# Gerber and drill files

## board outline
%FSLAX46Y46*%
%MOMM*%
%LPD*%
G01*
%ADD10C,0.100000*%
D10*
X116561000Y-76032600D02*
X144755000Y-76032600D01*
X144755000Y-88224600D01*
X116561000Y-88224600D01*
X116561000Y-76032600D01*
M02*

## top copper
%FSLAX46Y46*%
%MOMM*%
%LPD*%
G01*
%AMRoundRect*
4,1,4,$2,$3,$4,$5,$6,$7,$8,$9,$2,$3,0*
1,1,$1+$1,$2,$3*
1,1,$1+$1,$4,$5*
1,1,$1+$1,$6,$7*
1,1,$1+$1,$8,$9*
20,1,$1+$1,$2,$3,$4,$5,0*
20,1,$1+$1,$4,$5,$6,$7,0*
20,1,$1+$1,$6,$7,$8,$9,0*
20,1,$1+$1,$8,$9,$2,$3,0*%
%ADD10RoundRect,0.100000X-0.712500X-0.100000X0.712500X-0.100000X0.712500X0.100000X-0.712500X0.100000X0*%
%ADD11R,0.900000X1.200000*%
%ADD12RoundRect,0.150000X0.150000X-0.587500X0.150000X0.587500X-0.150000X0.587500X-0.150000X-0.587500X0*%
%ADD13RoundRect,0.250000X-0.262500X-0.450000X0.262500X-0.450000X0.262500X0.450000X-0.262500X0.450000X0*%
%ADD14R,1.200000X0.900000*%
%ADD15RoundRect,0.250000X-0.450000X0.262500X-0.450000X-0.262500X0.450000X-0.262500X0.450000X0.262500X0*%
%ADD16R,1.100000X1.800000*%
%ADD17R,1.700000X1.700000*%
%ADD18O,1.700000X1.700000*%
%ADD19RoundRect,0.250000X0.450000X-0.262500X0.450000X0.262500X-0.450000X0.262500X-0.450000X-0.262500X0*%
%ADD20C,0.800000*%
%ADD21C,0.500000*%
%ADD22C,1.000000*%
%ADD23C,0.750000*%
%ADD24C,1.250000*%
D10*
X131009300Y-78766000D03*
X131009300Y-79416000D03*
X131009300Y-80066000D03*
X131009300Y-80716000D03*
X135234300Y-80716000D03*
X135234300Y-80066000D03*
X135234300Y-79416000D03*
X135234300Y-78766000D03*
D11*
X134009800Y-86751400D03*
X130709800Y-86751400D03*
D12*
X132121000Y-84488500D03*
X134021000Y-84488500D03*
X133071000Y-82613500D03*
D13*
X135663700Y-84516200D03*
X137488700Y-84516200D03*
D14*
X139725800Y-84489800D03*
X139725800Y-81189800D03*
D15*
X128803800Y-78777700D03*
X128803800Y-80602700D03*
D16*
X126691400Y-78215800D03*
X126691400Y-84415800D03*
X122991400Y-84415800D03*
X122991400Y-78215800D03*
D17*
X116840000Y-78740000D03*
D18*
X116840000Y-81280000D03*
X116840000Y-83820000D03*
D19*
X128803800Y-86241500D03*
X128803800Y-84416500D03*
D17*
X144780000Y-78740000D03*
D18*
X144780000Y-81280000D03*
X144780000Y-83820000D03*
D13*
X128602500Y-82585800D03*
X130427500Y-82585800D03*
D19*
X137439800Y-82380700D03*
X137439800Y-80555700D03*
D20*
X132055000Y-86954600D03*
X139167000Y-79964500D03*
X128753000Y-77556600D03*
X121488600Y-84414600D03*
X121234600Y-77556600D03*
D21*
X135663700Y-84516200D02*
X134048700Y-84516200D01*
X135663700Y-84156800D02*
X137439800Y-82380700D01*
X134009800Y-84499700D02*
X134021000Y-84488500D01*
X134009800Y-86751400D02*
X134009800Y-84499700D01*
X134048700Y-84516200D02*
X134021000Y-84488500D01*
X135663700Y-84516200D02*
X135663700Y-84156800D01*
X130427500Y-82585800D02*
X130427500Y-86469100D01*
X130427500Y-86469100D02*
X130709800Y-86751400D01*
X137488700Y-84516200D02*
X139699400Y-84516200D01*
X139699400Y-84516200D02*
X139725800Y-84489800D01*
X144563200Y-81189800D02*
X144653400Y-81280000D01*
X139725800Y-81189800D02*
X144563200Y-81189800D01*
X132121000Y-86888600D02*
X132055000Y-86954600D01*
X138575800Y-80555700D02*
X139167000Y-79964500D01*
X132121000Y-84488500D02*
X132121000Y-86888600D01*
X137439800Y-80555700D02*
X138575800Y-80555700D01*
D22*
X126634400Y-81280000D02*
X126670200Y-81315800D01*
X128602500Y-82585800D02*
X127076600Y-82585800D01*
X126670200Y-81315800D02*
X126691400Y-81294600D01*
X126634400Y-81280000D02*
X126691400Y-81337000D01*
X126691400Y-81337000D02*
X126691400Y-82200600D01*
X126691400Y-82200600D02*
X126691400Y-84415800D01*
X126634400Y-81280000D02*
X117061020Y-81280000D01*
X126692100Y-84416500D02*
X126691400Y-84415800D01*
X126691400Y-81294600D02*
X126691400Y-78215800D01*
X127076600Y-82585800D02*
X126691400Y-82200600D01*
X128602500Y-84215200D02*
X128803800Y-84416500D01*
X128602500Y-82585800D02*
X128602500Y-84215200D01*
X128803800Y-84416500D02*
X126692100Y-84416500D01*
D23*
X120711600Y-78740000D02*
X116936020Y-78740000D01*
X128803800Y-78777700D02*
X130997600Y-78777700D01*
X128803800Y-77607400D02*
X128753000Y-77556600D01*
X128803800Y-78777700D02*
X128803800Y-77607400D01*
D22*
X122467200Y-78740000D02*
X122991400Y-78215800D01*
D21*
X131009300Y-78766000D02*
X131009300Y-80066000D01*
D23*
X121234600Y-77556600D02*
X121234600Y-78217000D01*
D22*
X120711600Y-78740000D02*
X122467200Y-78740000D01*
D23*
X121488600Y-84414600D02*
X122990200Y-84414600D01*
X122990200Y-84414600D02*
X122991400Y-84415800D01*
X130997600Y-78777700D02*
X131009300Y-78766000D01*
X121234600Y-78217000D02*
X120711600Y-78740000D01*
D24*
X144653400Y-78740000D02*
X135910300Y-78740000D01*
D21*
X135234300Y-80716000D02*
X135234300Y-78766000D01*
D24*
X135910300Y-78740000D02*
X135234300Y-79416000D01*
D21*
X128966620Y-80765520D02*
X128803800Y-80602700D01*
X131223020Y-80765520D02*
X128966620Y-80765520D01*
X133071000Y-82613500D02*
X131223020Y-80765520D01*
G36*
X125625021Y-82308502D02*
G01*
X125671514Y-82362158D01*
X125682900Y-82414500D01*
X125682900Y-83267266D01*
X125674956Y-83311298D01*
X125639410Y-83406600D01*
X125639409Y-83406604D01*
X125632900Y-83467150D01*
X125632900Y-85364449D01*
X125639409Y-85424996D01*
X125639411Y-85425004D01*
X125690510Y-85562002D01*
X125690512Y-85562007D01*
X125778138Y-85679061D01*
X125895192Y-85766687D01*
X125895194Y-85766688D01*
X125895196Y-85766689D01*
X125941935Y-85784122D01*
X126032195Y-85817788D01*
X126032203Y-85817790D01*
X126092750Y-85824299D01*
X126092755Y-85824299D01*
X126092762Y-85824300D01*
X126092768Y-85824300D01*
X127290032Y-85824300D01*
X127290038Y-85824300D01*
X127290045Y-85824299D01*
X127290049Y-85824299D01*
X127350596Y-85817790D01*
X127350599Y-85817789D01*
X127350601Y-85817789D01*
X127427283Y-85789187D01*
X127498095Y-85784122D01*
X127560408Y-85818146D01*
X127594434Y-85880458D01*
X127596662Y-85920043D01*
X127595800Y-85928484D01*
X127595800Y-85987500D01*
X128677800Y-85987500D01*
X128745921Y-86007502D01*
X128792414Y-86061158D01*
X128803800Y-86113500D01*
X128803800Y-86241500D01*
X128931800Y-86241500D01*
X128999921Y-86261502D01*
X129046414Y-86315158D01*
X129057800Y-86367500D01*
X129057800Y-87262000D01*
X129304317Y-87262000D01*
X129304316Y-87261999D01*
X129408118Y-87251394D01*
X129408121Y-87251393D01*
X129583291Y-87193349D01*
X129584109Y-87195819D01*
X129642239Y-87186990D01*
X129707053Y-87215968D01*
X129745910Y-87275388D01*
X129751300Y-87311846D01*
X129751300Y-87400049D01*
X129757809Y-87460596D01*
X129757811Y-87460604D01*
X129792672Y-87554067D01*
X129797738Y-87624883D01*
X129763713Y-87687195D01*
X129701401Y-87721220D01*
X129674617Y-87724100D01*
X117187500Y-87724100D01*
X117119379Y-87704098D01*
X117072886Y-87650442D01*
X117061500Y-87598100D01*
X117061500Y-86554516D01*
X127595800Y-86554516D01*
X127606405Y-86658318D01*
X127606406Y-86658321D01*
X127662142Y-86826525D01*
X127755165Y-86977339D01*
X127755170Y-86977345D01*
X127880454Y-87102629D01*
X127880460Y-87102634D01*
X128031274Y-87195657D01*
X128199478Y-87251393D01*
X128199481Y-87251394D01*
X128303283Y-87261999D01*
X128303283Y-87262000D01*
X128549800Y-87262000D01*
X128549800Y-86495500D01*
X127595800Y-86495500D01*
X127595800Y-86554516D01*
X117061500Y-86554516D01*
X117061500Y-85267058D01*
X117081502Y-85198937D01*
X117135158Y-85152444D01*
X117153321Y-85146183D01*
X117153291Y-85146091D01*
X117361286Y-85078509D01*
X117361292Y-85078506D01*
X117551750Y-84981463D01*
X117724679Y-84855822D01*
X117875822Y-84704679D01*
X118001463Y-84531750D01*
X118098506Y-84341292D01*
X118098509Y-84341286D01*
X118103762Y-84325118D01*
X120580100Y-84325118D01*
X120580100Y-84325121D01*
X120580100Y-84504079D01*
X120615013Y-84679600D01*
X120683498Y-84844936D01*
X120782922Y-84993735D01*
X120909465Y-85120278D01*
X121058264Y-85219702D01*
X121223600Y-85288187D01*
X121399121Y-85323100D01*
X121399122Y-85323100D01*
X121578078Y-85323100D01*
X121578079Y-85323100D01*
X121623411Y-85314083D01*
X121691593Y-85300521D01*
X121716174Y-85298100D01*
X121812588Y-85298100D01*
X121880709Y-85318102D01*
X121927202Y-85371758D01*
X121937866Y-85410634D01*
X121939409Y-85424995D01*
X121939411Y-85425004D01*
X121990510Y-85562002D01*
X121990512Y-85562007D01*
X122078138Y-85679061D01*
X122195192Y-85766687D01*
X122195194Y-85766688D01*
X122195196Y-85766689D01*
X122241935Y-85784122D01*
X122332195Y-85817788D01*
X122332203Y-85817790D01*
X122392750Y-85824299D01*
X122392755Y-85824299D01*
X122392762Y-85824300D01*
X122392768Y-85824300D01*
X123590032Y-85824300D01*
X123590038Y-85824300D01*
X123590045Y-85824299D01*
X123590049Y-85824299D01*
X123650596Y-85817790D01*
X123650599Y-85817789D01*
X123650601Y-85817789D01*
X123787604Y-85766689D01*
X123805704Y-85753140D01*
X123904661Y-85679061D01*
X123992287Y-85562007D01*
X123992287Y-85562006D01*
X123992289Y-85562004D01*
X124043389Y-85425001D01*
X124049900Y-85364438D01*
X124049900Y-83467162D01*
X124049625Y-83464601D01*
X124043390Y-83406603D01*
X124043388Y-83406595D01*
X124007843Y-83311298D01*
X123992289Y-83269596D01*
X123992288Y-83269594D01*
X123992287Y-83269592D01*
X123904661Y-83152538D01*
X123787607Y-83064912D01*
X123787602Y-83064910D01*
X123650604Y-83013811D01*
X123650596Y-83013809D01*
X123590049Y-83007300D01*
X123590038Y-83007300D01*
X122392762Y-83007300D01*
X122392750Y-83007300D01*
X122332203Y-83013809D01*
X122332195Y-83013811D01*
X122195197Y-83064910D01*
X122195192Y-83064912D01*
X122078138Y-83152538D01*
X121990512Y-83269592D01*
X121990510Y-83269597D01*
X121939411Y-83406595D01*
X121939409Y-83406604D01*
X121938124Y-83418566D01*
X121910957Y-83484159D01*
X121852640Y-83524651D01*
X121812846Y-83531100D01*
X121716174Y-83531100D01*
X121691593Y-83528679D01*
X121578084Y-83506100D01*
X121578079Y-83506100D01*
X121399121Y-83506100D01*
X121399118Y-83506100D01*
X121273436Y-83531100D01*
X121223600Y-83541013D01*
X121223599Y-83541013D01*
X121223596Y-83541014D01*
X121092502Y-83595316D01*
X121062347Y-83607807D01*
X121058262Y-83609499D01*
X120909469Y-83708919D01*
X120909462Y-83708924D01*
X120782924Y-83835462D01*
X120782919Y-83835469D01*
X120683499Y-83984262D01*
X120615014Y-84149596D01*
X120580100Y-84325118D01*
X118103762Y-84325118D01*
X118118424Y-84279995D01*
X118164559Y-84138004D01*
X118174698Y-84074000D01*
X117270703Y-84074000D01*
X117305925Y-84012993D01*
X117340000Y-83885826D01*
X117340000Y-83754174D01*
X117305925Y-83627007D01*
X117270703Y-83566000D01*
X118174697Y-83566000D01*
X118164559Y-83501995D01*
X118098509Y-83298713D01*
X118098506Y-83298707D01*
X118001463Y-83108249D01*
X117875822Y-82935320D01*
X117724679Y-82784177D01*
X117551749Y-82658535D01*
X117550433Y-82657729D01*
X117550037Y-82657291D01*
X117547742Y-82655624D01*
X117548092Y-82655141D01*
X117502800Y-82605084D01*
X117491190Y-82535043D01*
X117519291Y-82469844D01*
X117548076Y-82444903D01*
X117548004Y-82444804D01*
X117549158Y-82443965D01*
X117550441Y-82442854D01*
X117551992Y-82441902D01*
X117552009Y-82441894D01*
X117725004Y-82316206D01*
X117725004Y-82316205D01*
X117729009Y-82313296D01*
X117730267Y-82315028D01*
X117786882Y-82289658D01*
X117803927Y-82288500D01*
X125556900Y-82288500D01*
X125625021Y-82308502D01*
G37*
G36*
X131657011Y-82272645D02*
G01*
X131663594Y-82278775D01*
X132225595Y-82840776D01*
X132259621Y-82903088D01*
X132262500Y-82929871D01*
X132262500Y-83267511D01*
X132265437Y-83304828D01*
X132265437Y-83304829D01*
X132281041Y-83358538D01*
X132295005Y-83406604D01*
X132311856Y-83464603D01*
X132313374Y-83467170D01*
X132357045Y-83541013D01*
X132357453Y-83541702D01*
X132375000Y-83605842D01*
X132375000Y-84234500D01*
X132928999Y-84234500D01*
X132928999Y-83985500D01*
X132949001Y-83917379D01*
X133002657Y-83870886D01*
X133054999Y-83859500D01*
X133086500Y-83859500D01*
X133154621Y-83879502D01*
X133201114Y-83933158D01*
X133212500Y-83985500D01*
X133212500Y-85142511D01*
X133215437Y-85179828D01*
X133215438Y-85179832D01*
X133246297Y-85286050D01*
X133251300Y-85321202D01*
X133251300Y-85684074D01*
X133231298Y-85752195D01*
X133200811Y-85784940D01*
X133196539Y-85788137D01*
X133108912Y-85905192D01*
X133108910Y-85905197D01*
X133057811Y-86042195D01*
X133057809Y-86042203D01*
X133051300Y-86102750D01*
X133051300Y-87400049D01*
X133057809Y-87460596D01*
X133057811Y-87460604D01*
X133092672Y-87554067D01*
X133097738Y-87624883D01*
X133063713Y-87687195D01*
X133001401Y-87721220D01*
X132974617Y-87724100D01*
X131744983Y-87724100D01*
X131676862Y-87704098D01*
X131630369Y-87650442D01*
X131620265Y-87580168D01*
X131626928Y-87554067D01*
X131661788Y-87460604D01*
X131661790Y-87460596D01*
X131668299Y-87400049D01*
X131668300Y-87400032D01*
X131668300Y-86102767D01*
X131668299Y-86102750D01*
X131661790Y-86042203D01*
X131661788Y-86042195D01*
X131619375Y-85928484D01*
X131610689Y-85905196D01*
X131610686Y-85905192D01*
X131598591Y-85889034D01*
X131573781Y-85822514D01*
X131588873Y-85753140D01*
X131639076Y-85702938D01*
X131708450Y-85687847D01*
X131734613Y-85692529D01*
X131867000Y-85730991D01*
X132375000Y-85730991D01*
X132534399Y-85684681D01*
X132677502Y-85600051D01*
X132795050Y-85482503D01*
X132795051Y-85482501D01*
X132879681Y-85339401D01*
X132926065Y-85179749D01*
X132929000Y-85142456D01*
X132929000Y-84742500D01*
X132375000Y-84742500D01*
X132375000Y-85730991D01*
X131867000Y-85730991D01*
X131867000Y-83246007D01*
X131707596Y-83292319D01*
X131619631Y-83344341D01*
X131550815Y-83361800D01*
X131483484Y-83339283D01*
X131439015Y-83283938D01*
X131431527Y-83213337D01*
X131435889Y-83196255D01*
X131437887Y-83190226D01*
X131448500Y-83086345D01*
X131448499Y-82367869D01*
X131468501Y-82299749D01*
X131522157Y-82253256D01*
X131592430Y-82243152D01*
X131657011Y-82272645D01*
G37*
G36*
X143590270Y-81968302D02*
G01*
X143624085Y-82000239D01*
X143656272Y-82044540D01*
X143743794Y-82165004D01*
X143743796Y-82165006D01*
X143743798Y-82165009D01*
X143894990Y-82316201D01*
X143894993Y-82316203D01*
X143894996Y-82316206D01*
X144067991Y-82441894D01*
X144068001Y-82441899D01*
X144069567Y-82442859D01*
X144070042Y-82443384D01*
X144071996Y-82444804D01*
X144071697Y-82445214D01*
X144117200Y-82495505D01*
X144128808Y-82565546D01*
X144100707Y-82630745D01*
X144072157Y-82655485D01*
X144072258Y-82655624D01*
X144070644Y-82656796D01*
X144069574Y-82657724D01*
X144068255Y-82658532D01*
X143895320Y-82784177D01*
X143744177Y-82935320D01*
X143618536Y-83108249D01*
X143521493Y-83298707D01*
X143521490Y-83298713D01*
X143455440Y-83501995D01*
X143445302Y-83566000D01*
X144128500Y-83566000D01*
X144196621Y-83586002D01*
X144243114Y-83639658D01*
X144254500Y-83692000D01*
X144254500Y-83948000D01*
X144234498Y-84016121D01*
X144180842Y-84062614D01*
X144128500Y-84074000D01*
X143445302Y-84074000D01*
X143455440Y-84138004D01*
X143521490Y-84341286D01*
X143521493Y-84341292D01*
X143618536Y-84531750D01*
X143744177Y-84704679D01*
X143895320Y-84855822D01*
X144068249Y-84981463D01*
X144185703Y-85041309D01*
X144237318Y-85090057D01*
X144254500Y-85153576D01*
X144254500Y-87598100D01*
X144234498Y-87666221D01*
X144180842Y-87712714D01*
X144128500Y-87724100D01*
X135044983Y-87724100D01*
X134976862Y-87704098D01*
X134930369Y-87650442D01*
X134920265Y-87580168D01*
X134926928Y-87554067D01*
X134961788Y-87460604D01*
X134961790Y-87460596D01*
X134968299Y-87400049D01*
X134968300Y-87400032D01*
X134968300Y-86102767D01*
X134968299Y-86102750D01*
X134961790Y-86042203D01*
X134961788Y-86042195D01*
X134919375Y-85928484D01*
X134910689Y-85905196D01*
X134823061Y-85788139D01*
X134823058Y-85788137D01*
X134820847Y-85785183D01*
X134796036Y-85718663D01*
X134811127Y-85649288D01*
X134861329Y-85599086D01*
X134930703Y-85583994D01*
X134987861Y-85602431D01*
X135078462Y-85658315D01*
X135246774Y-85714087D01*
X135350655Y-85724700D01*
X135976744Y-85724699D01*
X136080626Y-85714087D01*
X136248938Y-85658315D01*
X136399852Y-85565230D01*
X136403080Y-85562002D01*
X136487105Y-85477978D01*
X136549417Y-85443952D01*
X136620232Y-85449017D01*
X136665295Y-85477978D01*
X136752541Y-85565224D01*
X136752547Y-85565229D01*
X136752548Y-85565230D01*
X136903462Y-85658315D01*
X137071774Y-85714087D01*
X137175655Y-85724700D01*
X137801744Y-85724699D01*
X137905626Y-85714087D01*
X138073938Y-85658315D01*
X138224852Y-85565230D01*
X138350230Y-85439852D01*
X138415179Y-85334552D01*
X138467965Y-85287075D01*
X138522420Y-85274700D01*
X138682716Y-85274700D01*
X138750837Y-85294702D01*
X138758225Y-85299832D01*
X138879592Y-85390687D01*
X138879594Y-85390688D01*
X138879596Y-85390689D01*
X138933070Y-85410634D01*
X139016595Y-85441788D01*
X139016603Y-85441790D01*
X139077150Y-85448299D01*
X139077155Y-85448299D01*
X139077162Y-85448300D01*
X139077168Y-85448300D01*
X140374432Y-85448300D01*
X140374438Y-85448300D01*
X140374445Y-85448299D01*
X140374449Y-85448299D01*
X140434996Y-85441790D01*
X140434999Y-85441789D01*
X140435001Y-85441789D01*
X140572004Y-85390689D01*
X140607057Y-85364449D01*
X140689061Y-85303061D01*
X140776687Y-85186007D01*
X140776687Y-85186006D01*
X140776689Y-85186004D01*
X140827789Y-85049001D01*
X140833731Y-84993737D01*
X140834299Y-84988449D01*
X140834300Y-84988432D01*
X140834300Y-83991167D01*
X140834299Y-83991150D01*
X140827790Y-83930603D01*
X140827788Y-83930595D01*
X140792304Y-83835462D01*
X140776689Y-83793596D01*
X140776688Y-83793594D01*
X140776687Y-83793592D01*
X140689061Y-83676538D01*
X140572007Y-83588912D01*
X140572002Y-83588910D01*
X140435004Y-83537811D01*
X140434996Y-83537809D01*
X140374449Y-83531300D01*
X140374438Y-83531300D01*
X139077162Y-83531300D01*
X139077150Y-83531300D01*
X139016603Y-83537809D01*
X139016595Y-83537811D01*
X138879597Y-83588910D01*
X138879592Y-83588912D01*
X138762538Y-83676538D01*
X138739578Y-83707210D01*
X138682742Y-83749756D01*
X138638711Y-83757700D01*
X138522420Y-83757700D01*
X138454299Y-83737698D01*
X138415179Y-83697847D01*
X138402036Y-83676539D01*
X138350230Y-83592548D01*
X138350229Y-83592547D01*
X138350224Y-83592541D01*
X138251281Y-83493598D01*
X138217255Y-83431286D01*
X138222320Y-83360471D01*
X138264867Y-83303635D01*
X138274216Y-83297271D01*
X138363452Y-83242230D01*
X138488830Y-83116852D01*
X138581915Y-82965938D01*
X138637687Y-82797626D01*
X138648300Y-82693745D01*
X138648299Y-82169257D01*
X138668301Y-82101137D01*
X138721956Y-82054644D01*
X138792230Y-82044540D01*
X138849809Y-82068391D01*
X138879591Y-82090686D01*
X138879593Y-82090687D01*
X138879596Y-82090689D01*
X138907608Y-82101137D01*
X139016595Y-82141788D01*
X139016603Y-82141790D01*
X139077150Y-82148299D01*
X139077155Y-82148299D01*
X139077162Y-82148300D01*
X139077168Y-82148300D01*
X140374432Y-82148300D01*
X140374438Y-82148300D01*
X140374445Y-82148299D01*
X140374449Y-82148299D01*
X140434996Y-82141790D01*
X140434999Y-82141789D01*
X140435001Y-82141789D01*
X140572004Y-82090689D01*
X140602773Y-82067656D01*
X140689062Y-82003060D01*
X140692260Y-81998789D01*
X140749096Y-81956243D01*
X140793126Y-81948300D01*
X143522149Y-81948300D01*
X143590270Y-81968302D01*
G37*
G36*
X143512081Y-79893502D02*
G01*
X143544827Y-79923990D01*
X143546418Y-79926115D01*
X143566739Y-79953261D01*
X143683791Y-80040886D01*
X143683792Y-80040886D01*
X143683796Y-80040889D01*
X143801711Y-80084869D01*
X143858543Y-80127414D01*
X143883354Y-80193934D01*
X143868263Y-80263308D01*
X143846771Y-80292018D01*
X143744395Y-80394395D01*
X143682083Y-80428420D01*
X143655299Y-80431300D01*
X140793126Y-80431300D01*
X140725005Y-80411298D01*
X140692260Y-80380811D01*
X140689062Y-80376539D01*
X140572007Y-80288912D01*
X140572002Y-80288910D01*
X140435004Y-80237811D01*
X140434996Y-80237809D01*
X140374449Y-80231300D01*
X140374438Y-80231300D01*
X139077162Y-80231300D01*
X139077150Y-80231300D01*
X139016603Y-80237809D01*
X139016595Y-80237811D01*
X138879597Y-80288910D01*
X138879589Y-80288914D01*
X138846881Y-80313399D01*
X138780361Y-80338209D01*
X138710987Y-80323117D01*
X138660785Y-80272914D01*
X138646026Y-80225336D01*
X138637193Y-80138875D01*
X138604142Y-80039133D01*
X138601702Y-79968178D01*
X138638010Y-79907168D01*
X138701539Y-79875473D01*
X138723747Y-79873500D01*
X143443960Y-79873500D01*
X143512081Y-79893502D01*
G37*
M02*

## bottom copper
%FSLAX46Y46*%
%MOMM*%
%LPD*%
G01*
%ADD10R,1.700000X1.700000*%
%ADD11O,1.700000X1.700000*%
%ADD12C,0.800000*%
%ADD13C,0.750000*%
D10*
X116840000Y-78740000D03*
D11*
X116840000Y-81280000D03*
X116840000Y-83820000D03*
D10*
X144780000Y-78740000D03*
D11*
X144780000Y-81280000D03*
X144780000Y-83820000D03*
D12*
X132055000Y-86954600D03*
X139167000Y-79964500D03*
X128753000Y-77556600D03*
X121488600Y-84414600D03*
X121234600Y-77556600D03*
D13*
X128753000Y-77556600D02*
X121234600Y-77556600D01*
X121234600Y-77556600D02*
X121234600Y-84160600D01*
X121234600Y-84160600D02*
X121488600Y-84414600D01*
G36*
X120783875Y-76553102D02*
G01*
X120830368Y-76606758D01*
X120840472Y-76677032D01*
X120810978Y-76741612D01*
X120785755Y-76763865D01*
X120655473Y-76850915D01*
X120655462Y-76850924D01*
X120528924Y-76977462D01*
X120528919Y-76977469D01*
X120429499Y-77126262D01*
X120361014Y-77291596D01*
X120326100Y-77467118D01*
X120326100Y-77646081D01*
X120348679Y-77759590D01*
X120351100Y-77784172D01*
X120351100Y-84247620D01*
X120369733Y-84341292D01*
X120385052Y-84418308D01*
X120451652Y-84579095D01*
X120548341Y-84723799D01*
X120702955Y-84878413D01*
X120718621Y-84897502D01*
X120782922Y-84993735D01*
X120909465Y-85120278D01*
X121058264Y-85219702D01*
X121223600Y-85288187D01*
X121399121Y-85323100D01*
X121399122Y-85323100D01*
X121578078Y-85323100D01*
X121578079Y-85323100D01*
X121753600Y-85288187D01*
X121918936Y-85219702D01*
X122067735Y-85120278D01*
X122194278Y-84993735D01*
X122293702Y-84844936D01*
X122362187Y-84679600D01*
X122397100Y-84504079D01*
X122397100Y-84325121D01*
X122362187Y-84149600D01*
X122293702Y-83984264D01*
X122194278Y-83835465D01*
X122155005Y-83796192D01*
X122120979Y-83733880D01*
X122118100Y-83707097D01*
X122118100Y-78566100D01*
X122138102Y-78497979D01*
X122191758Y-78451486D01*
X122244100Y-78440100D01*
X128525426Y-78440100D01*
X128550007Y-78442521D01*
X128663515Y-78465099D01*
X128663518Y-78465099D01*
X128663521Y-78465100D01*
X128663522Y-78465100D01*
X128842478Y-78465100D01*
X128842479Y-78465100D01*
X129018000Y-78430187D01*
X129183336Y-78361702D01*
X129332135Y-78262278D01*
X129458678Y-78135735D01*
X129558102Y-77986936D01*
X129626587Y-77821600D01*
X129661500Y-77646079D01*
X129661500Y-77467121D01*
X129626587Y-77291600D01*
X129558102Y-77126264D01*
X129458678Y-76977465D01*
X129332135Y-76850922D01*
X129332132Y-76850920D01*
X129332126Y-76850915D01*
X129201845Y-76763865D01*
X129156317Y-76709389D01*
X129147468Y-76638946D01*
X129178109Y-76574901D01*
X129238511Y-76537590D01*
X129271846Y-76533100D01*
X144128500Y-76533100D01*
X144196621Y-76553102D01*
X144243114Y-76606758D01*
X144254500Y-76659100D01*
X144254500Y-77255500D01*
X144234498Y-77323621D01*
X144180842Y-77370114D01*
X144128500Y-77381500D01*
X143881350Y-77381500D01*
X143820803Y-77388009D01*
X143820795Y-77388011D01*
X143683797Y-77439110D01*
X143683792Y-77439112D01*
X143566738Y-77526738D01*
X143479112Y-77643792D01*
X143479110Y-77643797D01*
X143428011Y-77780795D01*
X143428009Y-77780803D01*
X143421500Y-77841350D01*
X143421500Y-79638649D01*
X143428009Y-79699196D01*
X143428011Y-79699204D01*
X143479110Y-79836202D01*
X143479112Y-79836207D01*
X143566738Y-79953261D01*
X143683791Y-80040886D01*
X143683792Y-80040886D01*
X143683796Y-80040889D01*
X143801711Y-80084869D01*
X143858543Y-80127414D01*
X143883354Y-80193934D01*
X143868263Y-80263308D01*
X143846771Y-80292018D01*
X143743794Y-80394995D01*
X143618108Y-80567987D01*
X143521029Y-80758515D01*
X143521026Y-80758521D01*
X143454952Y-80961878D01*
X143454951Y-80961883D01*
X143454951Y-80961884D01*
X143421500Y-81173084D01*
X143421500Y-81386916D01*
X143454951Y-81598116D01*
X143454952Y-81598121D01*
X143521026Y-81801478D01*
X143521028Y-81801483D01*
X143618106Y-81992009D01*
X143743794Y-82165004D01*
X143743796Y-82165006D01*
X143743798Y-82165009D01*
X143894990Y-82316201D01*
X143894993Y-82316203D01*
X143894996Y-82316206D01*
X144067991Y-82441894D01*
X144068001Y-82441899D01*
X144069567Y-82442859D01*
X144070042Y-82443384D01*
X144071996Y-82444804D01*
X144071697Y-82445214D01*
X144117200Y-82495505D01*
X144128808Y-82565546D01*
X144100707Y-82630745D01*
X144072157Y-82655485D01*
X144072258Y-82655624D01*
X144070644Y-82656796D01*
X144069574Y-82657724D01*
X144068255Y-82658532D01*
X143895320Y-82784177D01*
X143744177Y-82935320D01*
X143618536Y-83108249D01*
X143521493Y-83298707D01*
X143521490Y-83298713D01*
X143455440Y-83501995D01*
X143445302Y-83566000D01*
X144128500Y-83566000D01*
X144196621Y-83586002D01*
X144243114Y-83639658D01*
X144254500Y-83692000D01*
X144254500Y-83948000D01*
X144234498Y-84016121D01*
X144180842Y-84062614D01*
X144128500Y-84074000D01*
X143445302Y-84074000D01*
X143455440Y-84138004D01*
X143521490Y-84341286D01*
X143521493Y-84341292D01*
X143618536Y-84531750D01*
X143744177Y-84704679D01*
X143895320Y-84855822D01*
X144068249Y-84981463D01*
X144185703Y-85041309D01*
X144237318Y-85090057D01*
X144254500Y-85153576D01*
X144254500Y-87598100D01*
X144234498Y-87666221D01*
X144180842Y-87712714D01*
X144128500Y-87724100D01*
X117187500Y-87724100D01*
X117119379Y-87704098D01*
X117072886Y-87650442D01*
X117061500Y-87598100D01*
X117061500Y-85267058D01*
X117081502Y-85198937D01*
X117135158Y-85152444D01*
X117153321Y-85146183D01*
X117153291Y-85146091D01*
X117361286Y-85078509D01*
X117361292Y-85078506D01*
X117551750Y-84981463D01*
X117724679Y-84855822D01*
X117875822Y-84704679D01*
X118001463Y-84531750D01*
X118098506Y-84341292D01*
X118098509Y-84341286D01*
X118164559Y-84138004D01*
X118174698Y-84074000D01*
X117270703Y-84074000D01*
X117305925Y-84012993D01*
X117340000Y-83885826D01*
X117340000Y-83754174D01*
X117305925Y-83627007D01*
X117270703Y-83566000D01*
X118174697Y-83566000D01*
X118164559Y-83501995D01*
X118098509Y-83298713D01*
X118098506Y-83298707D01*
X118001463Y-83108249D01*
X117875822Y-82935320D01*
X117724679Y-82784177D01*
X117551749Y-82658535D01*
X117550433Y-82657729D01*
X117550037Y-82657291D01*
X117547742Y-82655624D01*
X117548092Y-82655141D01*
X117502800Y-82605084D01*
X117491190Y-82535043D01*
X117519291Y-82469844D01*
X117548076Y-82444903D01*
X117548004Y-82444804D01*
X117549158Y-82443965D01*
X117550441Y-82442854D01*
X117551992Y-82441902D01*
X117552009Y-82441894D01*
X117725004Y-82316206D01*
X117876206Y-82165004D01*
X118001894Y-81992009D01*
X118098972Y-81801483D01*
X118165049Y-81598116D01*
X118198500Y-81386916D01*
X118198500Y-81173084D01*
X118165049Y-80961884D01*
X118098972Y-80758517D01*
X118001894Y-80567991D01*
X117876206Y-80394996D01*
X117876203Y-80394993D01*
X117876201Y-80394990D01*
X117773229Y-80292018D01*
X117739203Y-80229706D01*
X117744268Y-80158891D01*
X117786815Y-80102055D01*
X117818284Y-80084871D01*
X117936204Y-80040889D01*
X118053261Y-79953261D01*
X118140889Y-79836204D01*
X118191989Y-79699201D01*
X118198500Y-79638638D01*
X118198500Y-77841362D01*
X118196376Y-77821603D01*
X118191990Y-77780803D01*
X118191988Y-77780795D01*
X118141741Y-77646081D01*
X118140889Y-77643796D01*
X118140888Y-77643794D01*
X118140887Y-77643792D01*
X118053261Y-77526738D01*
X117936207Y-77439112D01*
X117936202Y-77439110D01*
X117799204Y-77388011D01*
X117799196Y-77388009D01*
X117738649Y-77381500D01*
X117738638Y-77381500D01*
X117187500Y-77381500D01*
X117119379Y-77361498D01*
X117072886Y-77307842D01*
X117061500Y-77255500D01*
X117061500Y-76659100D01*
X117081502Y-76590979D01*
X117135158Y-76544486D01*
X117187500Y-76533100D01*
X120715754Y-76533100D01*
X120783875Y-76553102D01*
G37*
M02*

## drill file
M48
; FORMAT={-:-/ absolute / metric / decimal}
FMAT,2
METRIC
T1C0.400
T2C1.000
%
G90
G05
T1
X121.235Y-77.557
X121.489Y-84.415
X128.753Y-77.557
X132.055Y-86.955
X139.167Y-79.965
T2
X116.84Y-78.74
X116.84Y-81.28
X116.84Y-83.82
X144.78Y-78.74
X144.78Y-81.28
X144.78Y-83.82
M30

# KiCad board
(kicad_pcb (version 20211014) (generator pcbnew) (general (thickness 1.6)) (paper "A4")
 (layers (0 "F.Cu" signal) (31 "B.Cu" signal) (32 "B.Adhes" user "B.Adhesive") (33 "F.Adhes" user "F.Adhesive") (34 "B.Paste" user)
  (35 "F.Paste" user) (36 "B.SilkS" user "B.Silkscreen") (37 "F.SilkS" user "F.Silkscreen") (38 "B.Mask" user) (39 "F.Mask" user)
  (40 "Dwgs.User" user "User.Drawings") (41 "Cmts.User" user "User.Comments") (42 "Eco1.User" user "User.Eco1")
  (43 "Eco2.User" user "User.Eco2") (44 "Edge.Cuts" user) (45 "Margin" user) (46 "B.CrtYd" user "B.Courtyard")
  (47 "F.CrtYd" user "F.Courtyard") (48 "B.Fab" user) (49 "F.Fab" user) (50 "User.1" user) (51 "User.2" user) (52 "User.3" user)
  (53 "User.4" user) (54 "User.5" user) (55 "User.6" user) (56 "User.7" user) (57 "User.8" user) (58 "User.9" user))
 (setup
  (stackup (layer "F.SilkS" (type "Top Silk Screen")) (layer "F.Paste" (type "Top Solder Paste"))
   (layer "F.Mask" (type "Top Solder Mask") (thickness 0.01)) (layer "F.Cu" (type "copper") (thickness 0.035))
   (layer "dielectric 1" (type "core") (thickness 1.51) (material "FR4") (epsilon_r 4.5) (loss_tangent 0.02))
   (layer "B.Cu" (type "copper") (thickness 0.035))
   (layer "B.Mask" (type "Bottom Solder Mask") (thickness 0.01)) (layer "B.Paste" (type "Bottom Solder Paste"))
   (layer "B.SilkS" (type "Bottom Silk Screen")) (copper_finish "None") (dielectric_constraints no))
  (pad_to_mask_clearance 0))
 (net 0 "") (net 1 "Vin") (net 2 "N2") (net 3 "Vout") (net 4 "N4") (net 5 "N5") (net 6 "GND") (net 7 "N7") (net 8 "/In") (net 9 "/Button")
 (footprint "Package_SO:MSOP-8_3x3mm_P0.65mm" (layer "F.Cu") (at 133.1218 79.741)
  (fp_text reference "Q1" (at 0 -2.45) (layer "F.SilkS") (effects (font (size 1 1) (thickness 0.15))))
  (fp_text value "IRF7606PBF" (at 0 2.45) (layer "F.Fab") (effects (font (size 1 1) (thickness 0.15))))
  (pad "1" smd roundrect locked (at -2.1125 -0.975) (size 1.625 0.4) (layers "F.Cu" "F.Paste" "F.Mask") (roundrect_rratio 0.25)
   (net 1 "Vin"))
  (pad "2" smd roundrect locked (at -2.1125 -0.325) (size 1.625 0.4) (layers "F.Cu" "F.Paste" "F.Mask") (roundrect_rratio 0.25)
   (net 1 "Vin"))
  (pad "3" smd roundrect locked (at -2.1125 0.325) (size 1.625 0.4) (layers "F.Cu" "F.Paste" "F.Mask") (roundrect_rratio 0.25) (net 1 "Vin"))
  (pad "4" smd roundrect locked (at -2.1125 0.975) (size 1.625 0.4) (layers "F.Cu" "F.Paste" "F.Mask") (roundrect_rratio 0.25) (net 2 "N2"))
  (pad "5" smd roundrect locked (at 2.1125 0.975) (size 1.625 0.4) (layers "F.Cu" "F.Paste" "F.Mask") (roundrect_rratio 0.25) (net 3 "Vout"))
  (pad "6" smd roundrect locked (at 2.1125 0.325) (size 1.625 0.4) (layers "F.Cu" "F.Paste" "F.Mask") (roundrect_rratio 0.25) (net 3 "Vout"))
  (pad "7" smd roundrect locked (at 2.1125 -0.325) (size 1.625 0.4) (layers "F.Cu" "F.Paste" "F.Mask") (roundrect_rratio 0.25)
   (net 3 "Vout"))
  (pad "8" smd roundrect locked (at 2.1125 -0.975) (size 1.625 0.4) (layers "F.Cu" "F.Paste" "F.Mask") (roundrect_rratio 0.25)
   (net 3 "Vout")))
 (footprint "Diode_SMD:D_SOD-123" (layer "F.Cu") (at 132.3598 86.7514 180)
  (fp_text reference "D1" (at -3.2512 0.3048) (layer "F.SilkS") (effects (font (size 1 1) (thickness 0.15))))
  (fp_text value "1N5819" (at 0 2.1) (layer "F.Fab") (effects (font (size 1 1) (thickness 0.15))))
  (pad "1" smd rect locked (at -1.65 0 180) (size 0.9 1.2) (layers "F.Cu" "F.Paste" "F.Mask") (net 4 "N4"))
  (pad "2" smd rect locked (at 1.65 0 180) (size 0.9 1.2) (layers "F.Cu" "F.Paste" "F.Mask") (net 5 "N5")))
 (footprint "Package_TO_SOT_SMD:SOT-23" (layer "F.Cu") (at 133.071 83.551 90)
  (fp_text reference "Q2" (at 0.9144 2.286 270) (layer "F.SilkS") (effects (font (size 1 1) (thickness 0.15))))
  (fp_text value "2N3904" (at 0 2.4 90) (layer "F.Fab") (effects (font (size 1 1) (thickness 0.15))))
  (pad "1" smd roundrect locked (at -0.9375 -0.95 90) (size 1.475 0.6) (layers "F.Cu" "F.Paste" "F.Mask") (roundrect_rratio 0.25)
   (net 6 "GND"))
  (pad "2" smd roundrect locked (at -0.9375 0.95 90) (size 1.475 0.6) (layers "F.Cu" "F.Paste" "F.Mask") (roundrect_rratio 0.25)
   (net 4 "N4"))
  (pad "3" smd roundrect locked (at 0.9375 0 90) (size 1.475 0.6) (layers "F.Cu" "F.Paste" "F.Mask") (roundrect_rratio 0.25) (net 2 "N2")))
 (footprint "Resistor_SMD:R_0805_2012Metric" (layer "F.Cu") (at 136.5762 84.5162)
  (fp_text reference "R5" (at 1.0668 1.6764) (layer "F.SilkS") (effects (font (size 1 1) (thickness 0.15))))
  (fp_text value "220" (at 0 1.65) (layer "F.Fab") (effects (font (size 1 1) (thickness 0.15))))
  (pad "1" smd roundrect locked (at -0.9125 0) (size 1.025 1.4) (layers "F.Cu" "F.Paste" "F.Mask") (roundrect_rratio 0.243902) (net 4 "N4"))
  (pad "2" smd roundrect locked (at 0.9125 0) (size 1.025 1.4) (layers "F.Cu" "F.Paste" "F.Mask") (roundrect_rratio 0.243902) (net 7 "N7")))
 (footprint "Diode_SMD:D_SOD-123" (layer "F.Cu") (at 139.7258 82.8398 90)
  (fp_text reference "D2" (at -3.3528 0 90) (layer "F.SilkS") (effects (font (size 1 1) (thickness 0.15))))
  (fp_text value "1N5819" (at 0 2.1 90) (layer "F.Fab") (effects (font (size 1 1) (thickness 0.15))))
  (pad "1" smd rect locked (at -1.65 0 90) (size 0.9 1.2) (layers "F.Cu" "F.Paste" "F.Mask") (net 7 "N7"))
  (pad "2" smd rect locked (at 1.65 0 90) (size 0.9 1.2) (layers "F.Cu" "F.Paste" "F.Mask") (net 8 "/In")))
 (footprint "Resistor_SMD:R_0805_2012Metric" (layer "F.Cu") (at 128.8038 79.6902 -90)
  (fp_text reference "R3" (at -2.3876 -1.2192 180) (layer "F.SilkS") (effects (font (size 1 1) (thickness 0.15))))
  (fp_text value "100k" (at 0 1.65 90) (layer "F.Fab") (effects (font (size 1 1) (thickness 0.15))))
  (pad "1" smd roundrect locked (at -0.9125 0 270) (size 1.025 1.4) (layers "F.Cu" "F.Paste" "F.Mask") (roundrect_rratio 0.243902)
   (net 1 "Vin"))
  (pad "2" smd roundrect locked (at 0.9125 0 270) (size 1.025 1.4) (layers "F.Cu" "F.Paste" "F.Mask") (roundrect_rratio 0.243902)
   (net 2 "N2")))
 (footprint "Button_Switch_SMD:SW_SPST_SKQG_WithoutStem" (layer "F.Cu") (at 124.8414 81.3158 -90)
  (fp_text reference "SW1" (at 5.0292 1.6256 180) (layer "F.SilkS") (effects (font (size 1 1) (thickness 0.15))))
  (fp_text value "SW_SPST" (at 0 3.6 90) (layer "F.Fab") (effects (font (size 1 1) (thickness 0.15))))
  (pad "1" smd rect locked (at -3.1 -1.85 270) (size 1.8 1.1) (layers "F.Cu" "F.Paste" "F.Mask") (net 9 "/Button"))
  (pad "1" smd rect locked (at 3.1 -1.85 270) (size 1.8 1.1) (layers "F.Cu" "F.Paste" "F.Mask") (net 9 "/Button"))
  (pad "2" smd rect locked (at 3.1 1.85 270) (size 1.8 1.1) (layers "F.Cu" "F.Paste" "F.Mask") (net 1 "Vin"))
  (pad "2" smd rect locked (at -3.1 1.85 270) (size 1.8 1.1) (layers "F.Cu" "F.Paste" "F.Mask") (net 1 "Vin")))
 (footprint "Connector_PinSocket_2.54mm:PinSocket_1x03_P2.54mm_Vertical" (layer "F.Cu") (at 116.84 78.74)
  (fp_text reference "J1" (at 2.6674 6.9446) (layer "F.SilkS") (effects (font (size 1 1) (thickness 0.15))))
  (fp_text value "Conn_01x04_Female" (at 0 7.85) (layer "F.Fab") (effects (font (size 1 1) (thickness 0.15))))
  (pad "1" thru_hole rect locked (at 0 0) (size 1.7 1.7) (drill 1) (layers *.Cu *.Mask) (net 1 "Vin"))
  (pad "2" thru_hole oval locked (at 0 2.54) (size 1.7 1.7) (drill 1) (layers *.Cu *.Mask) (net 9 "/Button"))
  (pad "3" thru_hole oval locked (at 0 5.08) (size 1.7 1.7) (drill 1) (layers *.Cu *.Mask) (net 6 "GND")))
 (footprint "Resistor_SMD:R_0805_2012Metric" (layer "F.Cu") (at 128.8038 85.329 90)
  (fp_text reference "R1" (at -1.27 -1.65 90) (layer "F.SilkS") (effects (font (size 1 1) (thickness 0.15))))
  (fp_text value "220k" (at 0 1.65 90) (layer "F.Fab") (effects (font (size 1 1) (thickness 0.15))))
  (pad "1" smd roundrect locked (at -0.9125 0 90) (size 1.025 1.4) (layers "F.Cu" "F.Paste" "F.Mask") (roundrect_rratio 0.243902)
   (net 6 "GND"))
  (pad "2" smd roundrect locked (at 0.9125 0 90) (size 1.025 1.4) (layers "F.Cu" "F.Paste" "F.Mask") (roundrect_rratio 0.243902)
   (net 9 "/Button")))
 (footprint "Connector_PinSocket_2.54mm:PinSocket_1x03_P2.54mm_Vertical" (layer "F.Cu") (at 144.78 78.74)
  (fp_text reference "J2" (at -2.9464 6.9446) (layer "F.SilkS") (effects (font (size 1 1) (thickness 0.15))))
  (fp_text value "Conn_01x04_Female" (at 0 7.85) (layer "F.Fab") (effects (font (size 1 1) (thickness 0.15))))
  (pad "1" thru_hole rect locked (at 0 0) (size 1.7 1.7) (drill 1) (layers *.Cu *.Mask) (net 3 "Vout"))
  (pad "2" thru_hole oval locked (at 0 2.54) (size 1.7 1.7) (drill 1) (layers *.Cu *.Mask) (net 8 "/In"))
  (pad "3" thru_hole oval locked (at 0 5.08) (size 1.7 1.7) (drill 1) (layers *.Cu *.Mask) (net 6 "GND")))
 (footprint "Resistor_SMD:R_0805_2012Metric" (layer "F.Cu") (at 129.515 82.5858)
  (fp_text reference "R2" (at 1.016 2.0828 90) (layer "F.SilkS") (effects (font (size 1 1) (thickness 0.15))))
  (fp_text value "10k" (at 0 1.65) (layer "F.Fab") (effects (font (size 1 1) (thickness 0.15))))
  (pad "1" smd roundrect locked (at -0.9125 0) (size 1.025 1.4) (layers "F.Cu" "F.Paste" "F.Mask") (roundrect_rratio 0.243902)
   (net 9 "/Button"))
  (pad "2" smd roundrect locked (at 0.9125 0) (size 1.025 1.4) (layers "F.Cu" "F.Paste" "F.Mask") (roundrect_rratio 0.243902) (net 5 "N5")))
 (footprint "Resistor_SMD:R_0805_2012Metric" (layer "F.Cu") (at 137.4398 81.4682 90)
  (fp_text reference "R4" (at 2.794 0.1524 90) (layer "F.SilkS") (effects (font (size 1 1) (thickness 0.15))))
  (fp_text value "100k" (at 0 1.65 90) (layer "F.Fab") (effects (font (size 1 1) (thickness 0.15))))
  (pad "1" smd roundrect locked (at -0.9125 0 90) (size 1.025 1.4) (layers "F.Cu" "F.Paste" "F.Mask") (roundrect_rratio 0.243902)
   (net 4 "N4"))
  (pad "2" smd roundrect locked (at 0.9125 0 90) (size 1.025 1.4) (layers "F.Cu" "F.Paste" "F.Mask") (roundrect_rratio 0.243902)
   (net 6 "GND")))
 (gr_rect (start 116.561 76.0326) (end 144.755 88.2246) (layer "Edge.Cuts") (width 0.1) (fill none))
 (segment (start 135.6637 84.5162) (end 134.0487 84.5162) (width 0.5) (layer "F.Cu") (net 4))
 (segment (start 135.6637 84.1568) (end 137.4398 82.3807) (width 0.5) (layer "F.Cu") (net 4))
 (segment (start 134.0098 84.4997) (end 134.021 84.4885) (width 0.5) (layer "F.Cu") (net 4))
 (segment (start 134.0098 86.7514) (end 134.0098 84.4997) (width 0.5) (layer "F.Cu") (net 4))
 (segment (start 134.0487 84.5162) (end 134.021 84.4885) (width 0.5) (layer "F.Cu") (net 4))
 (segment (start 135.6637 84.5162) (end 135.6637 84.1568) (width 0.5) (layer "F.Cu") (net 4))
 (segment (start 130.4275 82.5858) (end 130.4275 86.4691) (width 0.5) (layer "F.Cu") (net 5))
 (segment (start 130.4275 86.4691) (end 130.7098 86.7514) (width 0.5) (layer "F.Cu") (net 5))
 (segment (start 137.4887 84.5162) (end 139.6994 84.5162) (width 0.5) (layer "F.Cu") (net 7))
 (segment (start 139.6994 84.5162) (end 139.7258 84.4898) (width 0.5) (layer "F.Cu") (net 7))
 (segment (start 144.5632 81.1898) (end 144.6534 81.28) (width 0.5) (layer "F.Cu") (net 8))
 (segment (start 139.7258 81.1898) (end 144.5632 81.1898) (width 0.5) (layer "F.Cu") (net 8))
 (segment (start 132.121 86.8886) (end 132.055 86.9546) (width 0.5) (layer "F.Cu") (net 6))
 (segment (start 138.5758 80.5557) (end 139.167 79.9645) (width 0.5) (layer "F.Cu") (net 6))
 (segment (start 132.121 84.4885) (end 132.121 86.8886) (width 0.5) (layer "F.Cu") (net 6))
 (segment (start 137.4398 80.5557) (end 138.5758 80.5557) (width 0.5) (layer "F.Cu") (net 6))
 (via (at 132.055 86.9546) (size 0.8) (drill 0.4) (layers "F.Cu" "B.Cu") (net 6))
 (via (at 139.167 79.9645) (size 0.8) (drill 0.4) (layers "F.Cu" "B.Cu") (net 6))
 (segment (start 126.6344 81.28) (end 126.6702 81.3158) (width 1) (layer "F.Cu") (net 9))
 (segment (start 128.6025 82.5858) (end 127.0766 82.5858) (width 1) (layer "F.Cu") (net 9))
 (segment (start 126.6702 81.3158) (end 126.6914 81.2946) (width 1) (layer "F.Cu") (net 9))
 (segment (start 126.6344 81.28) (end 126.6914 81.337) (width 1) (layer "F.Cu") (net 9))
 (segment (start 126.6914 81.337) (end 126.6914 82.2006) (width 1) (layer "F.Cu") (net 9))
 (segment (start 126.6914 82.2006) (end 126.6914 84.4158) (width 1) (layer "F.Cu") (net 9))
 (segment (start 126.6344 81.28) (end 117.06102 81.28) (width 1) (layer "F.Cu") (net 9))
 (segment (start 126.6921 84.4165) (end 126.6914 84.4158) (width 1) (layer "F.Cu") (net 9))
 (segment (start 126.6914 81.2946) (end 126.6914 78.2158) (width 1) (layer "F.Cu") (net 9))
 (segment (start 127.0766 82.5858) (end 126.6914 82.2006) (width 1) (layer "F.Cu") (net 9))
 (segment (start 128.6025 84.2152) (end 128.8038 84.4165) (width 1) (layer "F.Cu") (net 9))
 (segment (start 128.6025 82.5858) (end 128.6025 84.2152) (width 1) (layer "F.Cu") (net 9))
 (segment (start 128.8038 84.4165) (end 126.6921 84.4165) (width 1) (layer "F.Cu") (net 9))
 (segment (start 120.7116 78.74) (end 116.93602 78.74) (width 0.75) (layer "F.Cu") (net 1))
 (segment (start 128.8038 78.7777) (end 130.9976 78.7777) (width 0.75) (layer "F.Cu") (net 1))
 (segment (start 128.8038 77.6074) (end 128.753 77.5566) (width 0.75) (layer "F.Cu") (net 1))
 (segment (start 128.8038 78.7777) (end 128.8038 77.6074) (width 0.75) (layer "F.Cu") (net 1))
 (segment (start 122.4672 78.74) (end 122.9914 78.2158) (width 1) (layer "F.Cu") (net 1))
 (segment (start 131.0093 78.766) (end 131.0093 80.066) (width 0.5) (layer "F.Cu") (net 1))
 (segment (start 121.2346 77.5566) (end 121.2346 78.217) (width 0.75) (layer "F.Cu") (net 1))
 (segment (start 120.7116 78.74) (end 122.4672 78.74) (width 1) (layer "F.Cu") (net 1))
 (segment (start 121.4886 84.4146) (end 122.9902 84.4146) (width 0.75) (layer "F.Cu") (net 1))
 (segment (start 122.9902 84.4146) (end 122.9914 84.4158) (width 0.75) (layer "F.Cu") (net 1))
 (segment (start 130.9976 78.7777) (end 131.0093 78.766) (width 0.75) (layer "F.Cu") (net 1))
 (segment (start 121.2346 78.217) (end 120.7116 78.74) (width 0.75) (layer "F.Cu") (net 1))
 (via (at 128.753 77.5566) (size 0.8) (drill 0.4) (layers "F.Cu" "B.Cu") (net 1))
 (via (at 121.4886 84.4146) (size 0.8) (drill 0.4) (layers "F.Cu" "B.Cu") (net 1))
 (via (at 121.2346 77.5566) (size 0.8) (drill 0.4) (layers "F.Cu" "B.Cu") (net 1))
 (segment (start 128.753 77.5566) (end 121.2346 77.5566) (width 0.75) (layer "B.Cu") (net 1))
 (segment (start 121.2346 77.5566) (end 121.2346 84.1606) (width 0.75) (layer "B.Cu") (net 1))
 (segment (start 121.2346 84.1606) (end 121.4886 84.4146) (width 0.75) (layer "B.Cu") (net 1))
 (segment (start 144.6534 78.74) (end 135.9103 78.74) (width 1.25) (layer "F.Cu") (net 3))
 (segment (start 135.2343 80.716) (end 135.2343 78.766) (width 0.5) (layer "F.Cu") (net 3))
 (segment (start 135.9103 78.74) (end 135.2343 79.416) (width 1.25) (layer "F.Cu") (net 3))
 (segment (start 128.96662 80.76552) (end 128.8038 80.6027) (width 0.5) (layer "F.Cu") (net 2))
 (segment (start 131.22302 80.76552) (end 128.96662 80.76552) (width 0.5) (layer "F.Cu") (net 2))
 (segment (start 133.071 82.6135) (end 131.22302 80.76552) (width 0.5) (layer "F.Cu") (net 2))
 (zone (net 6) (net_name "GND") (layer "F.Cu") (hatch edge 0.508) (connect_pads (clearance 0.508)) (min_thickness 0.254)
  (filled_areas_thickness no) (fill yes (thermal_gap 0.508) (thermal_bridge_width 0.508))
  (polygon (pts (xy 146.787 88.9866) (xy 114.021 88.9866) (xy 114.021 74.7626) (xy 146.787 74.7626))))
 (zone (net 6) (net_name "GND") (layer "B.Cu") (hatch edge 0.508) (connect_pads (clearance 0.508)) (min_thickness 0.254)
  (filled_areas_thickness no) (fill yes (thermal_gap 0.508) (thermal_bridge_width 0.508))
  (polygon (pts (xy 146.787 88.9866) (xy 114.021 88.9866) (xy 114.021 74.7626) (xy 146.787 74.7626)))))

